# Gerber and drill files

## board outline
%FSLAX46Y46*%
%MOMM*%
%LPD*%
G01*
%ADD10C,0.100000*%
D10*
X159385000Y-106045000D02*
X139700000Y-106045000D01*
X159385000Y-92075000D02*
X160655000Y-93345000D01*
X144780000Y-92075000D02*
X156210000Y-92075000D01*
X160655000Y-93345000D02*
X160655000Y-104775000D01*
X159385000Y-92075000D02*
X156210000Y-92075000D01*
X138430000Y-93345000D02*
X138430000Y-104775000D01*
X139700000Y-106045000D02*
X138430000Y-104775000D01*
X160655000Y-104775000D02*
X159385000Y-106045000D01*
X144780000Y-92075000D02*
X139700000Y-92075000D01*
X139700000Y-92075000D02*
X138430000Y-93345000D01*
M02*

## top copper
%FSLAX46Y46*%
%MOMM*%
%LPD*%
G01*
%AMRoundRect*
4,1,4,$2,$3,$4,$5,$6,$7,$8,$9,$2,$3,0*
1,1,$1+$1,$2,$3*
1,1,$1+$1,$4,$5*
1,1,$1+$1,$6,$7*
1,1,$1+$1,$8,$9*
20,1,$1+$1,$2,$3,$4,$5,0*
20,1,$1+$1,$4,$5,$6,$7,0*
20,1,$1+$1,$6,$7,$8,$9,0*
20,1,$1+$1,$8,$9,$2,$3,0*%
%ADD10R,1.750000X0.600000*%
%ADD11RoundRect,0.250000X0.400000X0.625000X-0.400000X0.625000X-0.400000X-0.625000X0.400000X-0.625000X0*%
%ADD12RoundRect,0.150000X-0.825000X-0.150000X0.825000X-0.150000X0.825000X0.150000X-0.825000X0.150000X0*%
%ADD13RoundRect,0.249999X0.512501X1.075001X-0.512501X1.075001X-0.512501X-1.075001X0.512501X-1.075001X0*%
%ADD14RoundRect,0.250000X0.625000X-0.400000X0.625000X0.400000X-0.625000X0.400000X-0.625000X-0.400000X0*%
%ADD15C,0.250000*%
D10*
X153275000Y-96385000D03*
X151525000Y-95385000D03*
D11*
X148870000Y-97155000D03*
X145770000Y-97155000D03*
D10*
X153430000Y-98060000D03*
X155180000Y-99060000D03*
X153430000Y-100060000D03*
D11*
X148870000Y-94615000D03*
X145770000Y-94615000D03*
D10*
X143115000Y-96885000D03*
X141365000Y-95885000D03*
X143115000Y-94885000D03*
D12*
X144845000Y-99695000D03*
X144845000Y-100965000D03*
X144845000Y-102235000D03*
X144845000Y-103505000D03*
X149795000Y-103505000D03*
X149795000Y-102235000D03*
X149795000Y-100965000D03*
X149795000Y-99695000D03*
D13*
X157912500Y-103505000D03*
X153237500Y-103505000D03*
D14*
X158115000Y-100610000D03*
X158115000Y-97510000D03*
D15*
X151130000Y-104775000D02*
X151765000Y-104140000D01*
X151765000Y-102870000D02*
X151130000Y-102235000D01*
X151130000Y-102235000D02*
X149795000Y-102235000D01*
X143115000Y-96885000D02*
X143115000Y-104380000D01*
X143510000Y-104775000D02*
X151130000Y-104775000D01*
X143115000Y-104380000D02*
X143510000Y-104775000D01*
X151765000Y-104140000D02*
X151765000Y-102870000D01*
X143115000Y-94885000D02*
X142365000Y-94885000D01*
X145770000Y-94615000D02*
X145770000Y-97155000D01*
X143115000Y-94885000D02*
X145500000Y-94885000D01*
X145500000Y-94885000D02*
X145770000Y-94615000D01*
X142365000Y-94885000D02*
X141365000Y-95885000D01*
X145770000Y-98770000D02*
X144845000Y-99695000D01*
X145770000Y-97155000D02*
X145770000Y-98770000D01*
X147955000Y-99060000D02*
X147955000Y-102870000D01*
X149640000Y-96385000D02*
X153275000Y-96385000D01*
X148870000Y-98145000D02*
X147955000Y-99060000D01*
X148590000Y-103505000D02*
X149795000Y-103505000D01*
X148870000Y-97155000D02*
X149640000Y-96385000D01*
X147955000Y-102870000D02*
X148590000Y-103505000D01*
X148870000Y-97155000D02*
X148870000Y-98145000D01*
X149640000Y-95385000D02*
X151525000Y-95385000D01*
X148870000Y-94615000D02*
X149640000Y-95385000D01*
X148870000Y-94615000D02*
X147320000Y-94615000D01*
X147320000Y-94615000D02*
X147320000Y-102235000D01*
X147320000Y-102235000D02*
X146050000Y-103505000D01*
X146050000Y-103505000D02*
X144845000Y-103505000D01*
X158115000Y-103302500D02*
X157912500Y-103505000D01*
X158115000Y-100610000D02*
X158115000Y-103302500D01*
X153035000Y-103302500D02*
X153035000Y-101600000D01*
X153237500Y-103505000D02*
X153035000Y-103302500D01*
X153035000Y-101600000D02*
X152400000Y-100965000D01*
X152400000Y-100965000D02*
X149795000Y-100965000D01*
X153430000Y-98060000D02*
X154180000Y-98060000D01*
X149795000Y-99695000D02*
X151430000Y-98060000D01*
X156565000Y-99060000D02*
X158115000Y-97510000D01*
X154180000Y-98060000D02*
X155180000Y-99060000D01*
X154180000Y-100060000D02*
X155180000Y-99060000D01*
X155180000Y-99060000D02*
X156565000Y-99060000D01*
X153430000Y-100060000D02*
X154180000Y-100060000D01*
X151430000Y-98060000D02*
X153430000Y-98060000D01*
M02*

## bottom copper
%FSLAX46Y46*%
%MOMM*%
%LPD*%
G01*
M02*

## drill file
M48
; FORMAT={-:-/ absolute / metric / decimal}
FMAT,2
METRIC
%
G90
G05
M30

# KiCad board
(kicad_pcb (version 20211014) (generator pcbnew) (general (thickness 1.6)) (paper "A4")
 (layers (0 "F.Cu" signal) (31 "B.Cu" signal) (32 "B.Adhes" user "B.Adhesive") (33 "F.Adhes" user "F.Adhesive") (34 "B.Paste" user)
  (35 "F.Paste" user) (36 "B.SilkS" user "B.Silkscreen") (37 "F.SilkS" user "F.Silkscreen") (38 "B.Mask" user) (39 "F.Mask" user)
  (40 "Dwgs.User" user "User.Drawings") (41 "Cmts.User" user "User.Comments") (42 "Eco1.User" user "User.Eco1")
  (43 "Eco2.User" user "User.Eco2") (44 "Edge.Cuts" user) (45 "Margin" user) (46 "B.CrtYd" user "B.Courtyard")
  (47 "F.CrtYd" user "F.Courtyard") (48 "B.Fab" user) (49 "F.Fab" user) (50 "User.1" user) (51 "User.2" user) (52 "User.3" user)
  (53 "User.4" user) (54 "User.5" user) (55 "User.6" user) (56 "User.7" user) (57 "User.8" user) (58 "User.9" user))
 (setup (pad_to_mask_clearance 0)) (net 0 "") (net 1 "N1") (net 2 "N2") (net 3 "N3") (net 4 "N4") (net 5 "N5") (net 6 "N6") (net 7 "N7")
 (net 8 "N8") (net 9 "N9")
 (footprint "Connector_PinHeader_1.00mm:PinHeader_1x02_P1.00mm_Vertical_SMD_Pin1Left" (layer "F.Cu") (at 152.4 95.885 180)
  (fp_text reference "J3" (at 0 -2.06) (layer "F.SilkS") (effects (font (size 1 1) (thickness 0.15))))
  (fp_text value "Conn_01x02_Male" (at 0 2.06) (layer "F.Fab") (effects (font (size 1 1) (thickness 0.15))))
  (pad "1" smd rect locked (at -0.875 -0.5 180) (size 1.75 0.6) (layers "F.Cu" "F.Paste" "F.Mask") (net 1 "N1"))
  (pad "2" smd rect locked (at 0.875 0.5 180) (size 1.75 0.6) (layers "F.Cu" "F.Paste" "F.Mask") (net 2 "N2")))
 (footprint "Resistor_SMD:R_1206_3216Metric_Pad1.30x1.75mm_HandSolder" (layer "F.Cu") (at 147.32 97.155 180)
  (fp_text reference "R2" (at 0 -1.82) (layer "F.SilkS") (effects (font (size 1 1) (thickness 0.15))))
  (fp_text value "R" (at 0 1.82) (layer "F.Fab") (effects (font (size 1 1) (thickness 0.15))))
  (pad "1" smd roundrect locked (at -1.55 0 180) (size 1.3 1.75) (layers "F.Cu" "F.Paste" "F.Mask") (roundrect_rratio 0.192308) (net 1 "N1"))
  (pad "2" smd roundrect locked (at 1.55 0 180) (size 1.3 1.75) (layers "F.Cu" "F.Paste" "F.Mask") (roundrect_rratio 0.192308) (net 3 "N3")))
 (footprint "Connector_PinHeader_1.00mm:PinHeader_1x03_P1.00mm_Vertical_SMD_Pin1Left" (layer "F.Cu") (at 154.305 99.06)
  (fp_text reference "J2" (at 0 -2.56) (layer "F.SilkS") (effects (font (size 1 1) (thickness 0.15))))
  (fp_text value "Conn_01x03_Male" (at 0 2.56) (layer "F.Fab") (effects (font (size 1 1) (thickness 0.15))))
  (pad "1" smd rect locked (at -0.875 -1) (size 1.75 0.6) (layers "F.Cu" "F.Paste" "F.Mask") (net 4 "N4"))
  (pad "2" smd rect locked (at 0.875 0) (size 1.75 0.6) (layers "F.Cu" "F.Paste" "F.Mask") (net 4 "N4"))
  (pad "3" smd rect locked (at -0.875 1) (size 1.75 0.6) (layers "F.Cu" "F.Paste" "F.Mask") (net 4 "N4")))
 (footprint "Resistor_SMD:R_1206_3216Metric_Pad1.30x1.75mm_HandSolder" (layer "F.Cu") (at 147.32 94.615 180)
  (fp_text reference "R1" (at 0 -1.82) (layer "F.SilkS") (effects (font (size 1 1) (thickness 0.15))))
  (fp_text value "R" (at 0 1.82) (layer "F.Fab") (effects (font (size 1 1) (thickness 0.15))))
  (pad "1" smd roundrect locked (at -1.55 0 180) (size 1.3 1.75) (layers "F.Cu" "F.Paste" "F.Mask") (roundrect_rratio 0.192308) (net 2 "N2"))
  (pad "2" smd roundrect locked (at 1.55 0 180) (size 1.3 1.75) (layers "F.Cu" "F.Paste" "F.Mask") (roundrect_rratio 0.192308) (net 3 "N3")))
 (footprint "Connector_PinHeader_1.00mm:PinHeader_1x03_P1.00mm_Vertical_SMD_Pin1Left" (layer "F.Cu") (at 142.24 95.885 180)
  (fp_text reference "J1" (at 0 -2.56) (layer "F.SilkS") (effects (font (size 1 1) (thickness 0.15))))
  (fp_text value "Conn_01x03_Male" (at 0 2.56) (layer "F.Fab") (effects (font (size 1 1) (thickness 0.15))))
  (pad "1" smd rect locked (at -0.875 -1 180) (size 1.75 0.6) (layers "F.Cu" "F.Paste" "F.Mask") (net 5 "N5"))
  (pad "2" smd rect locked (at 0.875 0 180) (size 1.75 0.6) (layers "F.Cu" "F.Paste" "F.Mask") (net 3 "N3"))
  (pad "3" smd rect locked (at -0.875 1 180) (size 1.75 0.6) (layers "F.Cu" "F.Paste" "F.Mask") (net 3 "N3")))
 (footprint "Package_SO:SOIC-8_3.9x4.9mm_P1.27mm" (layer "F.Cu") (at 147.32 101.6)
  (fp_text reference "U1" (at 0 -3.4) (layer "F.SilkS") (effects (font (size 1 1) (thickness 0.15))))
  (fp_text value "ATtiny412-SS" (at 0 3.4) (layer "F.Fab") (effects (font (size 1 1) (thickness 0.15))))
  (pad "1" smd roundrect locked (at -2.475 -1.905) (size 1.95 0.6) (layers "F.Cu" "F.Paste" "F.Mask") (roundrect_rratio 0.25) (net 3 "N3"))
  (pad "2" smd roundrect locked (at -2.475 -0.635) (size 1.95 0.6) (layers "F.Cu" "F.Paste" "F.Mask") (roundrect_rratio 0.25) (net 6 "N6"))
  (pad "3" smd roundrect locked (at -2.475 0.635) (size 1.95 0.6) (layers "F.Cu" "F.Paste" "F.Mask") (roundrect_rratio 0.25) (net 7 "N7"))
  (pad "4" smd roundrect locked (at -2.475 1.905) (size 1.95 0.6) (layers "F.Cu" "F.Paste" "F.Mask") (roundrect_rratio 0.25) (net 2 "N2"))
  (pad "5" smd roundrect locked (at 2.475 1.905) (size 1.95 0.6) (layers "F.Cu" "F.Paste" "F.Mask") (roundrect_rratio 0.25) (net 1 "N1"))
  (pad "6" smd roundrect locked (at 2.475 0.635) (size 1.95 0.6) (layers "F.Cu" "F.Paste" "F.Mask") (roundrect_rratio 0.25) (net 5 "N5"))
  (pad "7" smd roundrect locked (at 2.475 -0.635) (size 1.95 0.6) (layers "F.Cu" "F.Paste" "F.Mask") (roundrect_rratio 0.25) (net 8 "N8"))
  (pad "8" smd roundrect locked (at 2.475 -1.905) (size 1.95 0.6) (layers "F.Cu" "F.Paste" "F.Mask") (roundrect_rratio 0.25) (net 4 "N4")))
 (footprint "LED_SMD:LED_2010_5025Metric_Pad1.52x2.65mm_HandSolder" (layer "F.Cu") (at 155.575 103.505 180)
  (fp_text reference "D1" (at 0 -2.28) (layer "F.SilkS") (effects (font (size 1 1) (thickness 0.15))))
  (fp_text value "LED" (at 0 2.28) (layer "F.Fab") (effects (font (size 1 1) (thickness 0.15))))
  (pad "1" smd roundrect locked (at -2.3375 0 180) (size 1.525 2.65) (layers "F.Cu" "F.Paste" "F.Mask") (roundrect_rratio 0.163934)
   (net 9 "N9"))
  (pad "2" smd roundrect locked (at 2.3375 0 180) (size 1.525 2.65) (layers "F.Cu" "F.Paste" "F.Mask") (roundrect_rratio 0.163934)
   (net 8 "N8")))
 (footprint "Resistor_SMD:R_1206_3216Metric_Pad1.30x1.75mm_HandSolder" (layer "F.Cu") (at 158.115 99.06 90)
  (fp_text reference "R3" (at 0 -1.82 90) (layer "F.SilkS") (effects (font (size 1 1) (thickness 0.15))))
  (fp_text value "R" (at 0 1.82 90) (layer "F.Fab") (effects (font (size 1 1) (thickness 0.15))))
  (pad "1" smd roundrect locked (at -1.55 0 90) (size 1.3 1.75) (layers "F.Cu" "F.Paste" "F.Mask") (roundrect_rratio 0.192308) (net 9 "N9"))
  (pad "2" smd roundrect locked (at 1.55 0 90) (size 1.3 1.75) (layers "F.Cu" "F.Paste" "F.Mask") (roundrect_rratio 0.192308) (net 4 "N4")))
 (gr_line (start 159.385 106.045) (end 139.7 106.045) (layer "Edge.Cuts") (width 0.1))
 (gr_line (start 159.385 92.075) (end 160.655 93.345) (layer "Edge.Cuts") (width 0.1))
 (gr_line (start 144.78 92.075) (end 156.21 92.075) (layer "Edge.Cuts") (width 0.1))
 (gr_line (start 160.655 93.345) (end 160.655 104.775) (layer "Edge.Cuts") (width 0.1))
 (gr_line (start 159.385 92.075) (end 156.21 92.075) (layer "Edge.Cuts") (width 0.1))
 (gr_line (start 138.43 93.345) (end 138.43 104.775) (layer "Edge.Cuts") (width 0.1))
 (gr_line (start 139.7 106.045) (end 138.43 104.775) (layer "Edge.Cuts") (width 0.1))
 (gr_line (start 160.655 104.775) (end 159.385 106.045) (layer "Edge.Cuts") (width 0.1))
 (gr_line (start 144.78 92.075) (end 139.7 92.075) (layer "Edge.Cuts") (width 0.1))
 (gr_line (start 139.7 92.075) (end 138.43 93.345) (layer "Edge.Cuts") (width 0.1))
 (segment (start 151.13 104.775) (end 151.765 104.14) (width 0.25) (layer "F.Cu") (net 5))
 (segment (start 151.765 102.87) (end 151.13 102.235) (width 0.25) (layer "F.Cu") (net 5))
 (segment (start 151.13 102.235) (end 149.795 102.235) (width 0.25) (layer "F.Cu") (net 5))
 (segment (start 143.115 96.885) (end 143.115 104.38) (width 0.25) (layer "F.Cu") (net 5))
 (segment (start 143.51 104.775) (end 151.13 104.775) (width 0.25) (layer "F.Cu") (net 5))
 (segment (start 143.115 104.38) (end 143.51 104.775) (width 0.25) (layer "F.Cu") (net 5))
 (segment (start 151.765 104.14) (end 151.765 102.87) (width 0.25) (layer "F.Cu") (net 5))
 (segment (start 143.115 94.885) (end 142.365 94.885) (width 0.25) (layer "F.Cu") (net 3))
 (segment (start 145.77 94.615) (end 145.77 97.155) (width 0.25) (layer "F.Cu") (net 3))
 (segment (start 143.115 94.885) (end 145.5 94.885) (width 0.25) (layer "F.Cu") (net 3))
 (segment (start 145.5 94.885) (end 145.77 94.615) (width 0.25) (layer "F.Cu") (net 3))
 (segment (start 142.365 94.885) (end 141.365 95.885) (width 0.25) (layer "F.Cu") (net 3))
 (segment (start 145.77 98.77) (end 144.845 99.695) (width 0.25) (layer "F.Cu") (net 3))
 (segment (start 145.77 97.155) (end 145.77 98.77) (width 0.25) (layer "F.Cu") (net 3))
 (segment (start 147.955 99.06) (end 147.955 102.87) (width 0.25) (layer "F.Cu") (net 1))
 (segment (start 149.64 96.385) (end 153.275 96.385) (width 0.25) (layer "F.Cu") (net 1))
 (segment (start 148.87 98.145) (end 147.955 99.06) (width 0.25) (layer "F.Cu") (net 1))
 (segment (start 148.59 103.505) (end 149.795 103.505) (width 0.25) (layer "F.Cu") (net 1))
 (segment (start 148.87 97.155) (end 149.64 96.385) (width 0.25) (layer "F.Cu") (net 1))
 (segment (start 147.955 102.87) (end 148.59 103.505) (width 0.25) (layer "F.Cu") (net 1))
 (segment (start 148.87 97.155) (end 148.87 98.145) (width 0.25) (layer "F.Cu") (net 1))
 (segment (start 149.64 95.385) (end 151.525 95.385) (width 0.25) (layer "F.Cu") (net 2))
 (segment (start 148.87 94.615) (end 149.64 95.385) (width 0.25) (layer "F.Cu") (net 2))
 (segment (start 148.87 94.615) (end 147.32 94.615) (width 0.25) (layer "F.Cu") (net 2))
 (segment (start 147.32 94.615) (end 147.32 102.235) (width 0.25) (layer "F.Cu") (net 2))
 (segment (start 147.32 102.235) (end 146.05 103.505) (width 0.25) (layer "F.Cu") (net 2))
 (segment (start 146.05 103.505) (end 144.845 103.505) (width 0.25) (layer "F.Cu") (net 2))
 (segment (start 158.115 103.3025) (end 157.9125 103.505) (width 0.25) (layer "F.Cu") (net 9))
 (segment (start 158.115 100.61) (end 158.115 103.3025) (width 0.25) (layer "F.Cu") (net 9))
 (segment (start 153.035 103.3025) (end 153.035 101.6) (width 0.25) (layer "F.Cu") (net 8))
 (segment (start 153.2375 103.505) (end 153.035 103.3025) (width 0.25) (layer "F.Cu") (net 8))
 (segment (start 153.035 101.6) (end 152.4 100.965) (width 0.25) (layer "F.Cu") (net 8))
 (segment (start 152.4 100.965) (end 149.795 100.965) (width 0.25) (layer "F.Cu") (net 8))
 (segment (start 153.43 98.06) (end 154.18 98.06) (width 0.25) (layer "F.Cu") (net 4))
 (segment (start 149.795 99.695) (end 151.43 98.06) (width 0.25) (layer "F.Cu") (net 4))
 (segment (start 156.565 99.06) (end 158.115 97.51) (width 0.25) (layer "F.Cu") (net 4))
 (segment (start 154.18 98.06) (end 155.18 99.06) (width 0.25) (layer "F.Cu") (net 4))
 (segment (start 154.18 100.06) (end 155.18 99.06) (width 0.25) (layer "F.Cu") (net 4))
 (segment (start 155.18 99.06) (end 156.565 99.06) (width 0.25) (layer "F.Cu") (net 4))
 (segment (start 153.43 100.06) (end 154.18 100.06) (width 0.25) (layer "F.Cu") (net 4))
 (segment (start 151.43 98.06) (end 153.43 98.06) (width 0.25) (layer "F.Cu") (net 4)))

